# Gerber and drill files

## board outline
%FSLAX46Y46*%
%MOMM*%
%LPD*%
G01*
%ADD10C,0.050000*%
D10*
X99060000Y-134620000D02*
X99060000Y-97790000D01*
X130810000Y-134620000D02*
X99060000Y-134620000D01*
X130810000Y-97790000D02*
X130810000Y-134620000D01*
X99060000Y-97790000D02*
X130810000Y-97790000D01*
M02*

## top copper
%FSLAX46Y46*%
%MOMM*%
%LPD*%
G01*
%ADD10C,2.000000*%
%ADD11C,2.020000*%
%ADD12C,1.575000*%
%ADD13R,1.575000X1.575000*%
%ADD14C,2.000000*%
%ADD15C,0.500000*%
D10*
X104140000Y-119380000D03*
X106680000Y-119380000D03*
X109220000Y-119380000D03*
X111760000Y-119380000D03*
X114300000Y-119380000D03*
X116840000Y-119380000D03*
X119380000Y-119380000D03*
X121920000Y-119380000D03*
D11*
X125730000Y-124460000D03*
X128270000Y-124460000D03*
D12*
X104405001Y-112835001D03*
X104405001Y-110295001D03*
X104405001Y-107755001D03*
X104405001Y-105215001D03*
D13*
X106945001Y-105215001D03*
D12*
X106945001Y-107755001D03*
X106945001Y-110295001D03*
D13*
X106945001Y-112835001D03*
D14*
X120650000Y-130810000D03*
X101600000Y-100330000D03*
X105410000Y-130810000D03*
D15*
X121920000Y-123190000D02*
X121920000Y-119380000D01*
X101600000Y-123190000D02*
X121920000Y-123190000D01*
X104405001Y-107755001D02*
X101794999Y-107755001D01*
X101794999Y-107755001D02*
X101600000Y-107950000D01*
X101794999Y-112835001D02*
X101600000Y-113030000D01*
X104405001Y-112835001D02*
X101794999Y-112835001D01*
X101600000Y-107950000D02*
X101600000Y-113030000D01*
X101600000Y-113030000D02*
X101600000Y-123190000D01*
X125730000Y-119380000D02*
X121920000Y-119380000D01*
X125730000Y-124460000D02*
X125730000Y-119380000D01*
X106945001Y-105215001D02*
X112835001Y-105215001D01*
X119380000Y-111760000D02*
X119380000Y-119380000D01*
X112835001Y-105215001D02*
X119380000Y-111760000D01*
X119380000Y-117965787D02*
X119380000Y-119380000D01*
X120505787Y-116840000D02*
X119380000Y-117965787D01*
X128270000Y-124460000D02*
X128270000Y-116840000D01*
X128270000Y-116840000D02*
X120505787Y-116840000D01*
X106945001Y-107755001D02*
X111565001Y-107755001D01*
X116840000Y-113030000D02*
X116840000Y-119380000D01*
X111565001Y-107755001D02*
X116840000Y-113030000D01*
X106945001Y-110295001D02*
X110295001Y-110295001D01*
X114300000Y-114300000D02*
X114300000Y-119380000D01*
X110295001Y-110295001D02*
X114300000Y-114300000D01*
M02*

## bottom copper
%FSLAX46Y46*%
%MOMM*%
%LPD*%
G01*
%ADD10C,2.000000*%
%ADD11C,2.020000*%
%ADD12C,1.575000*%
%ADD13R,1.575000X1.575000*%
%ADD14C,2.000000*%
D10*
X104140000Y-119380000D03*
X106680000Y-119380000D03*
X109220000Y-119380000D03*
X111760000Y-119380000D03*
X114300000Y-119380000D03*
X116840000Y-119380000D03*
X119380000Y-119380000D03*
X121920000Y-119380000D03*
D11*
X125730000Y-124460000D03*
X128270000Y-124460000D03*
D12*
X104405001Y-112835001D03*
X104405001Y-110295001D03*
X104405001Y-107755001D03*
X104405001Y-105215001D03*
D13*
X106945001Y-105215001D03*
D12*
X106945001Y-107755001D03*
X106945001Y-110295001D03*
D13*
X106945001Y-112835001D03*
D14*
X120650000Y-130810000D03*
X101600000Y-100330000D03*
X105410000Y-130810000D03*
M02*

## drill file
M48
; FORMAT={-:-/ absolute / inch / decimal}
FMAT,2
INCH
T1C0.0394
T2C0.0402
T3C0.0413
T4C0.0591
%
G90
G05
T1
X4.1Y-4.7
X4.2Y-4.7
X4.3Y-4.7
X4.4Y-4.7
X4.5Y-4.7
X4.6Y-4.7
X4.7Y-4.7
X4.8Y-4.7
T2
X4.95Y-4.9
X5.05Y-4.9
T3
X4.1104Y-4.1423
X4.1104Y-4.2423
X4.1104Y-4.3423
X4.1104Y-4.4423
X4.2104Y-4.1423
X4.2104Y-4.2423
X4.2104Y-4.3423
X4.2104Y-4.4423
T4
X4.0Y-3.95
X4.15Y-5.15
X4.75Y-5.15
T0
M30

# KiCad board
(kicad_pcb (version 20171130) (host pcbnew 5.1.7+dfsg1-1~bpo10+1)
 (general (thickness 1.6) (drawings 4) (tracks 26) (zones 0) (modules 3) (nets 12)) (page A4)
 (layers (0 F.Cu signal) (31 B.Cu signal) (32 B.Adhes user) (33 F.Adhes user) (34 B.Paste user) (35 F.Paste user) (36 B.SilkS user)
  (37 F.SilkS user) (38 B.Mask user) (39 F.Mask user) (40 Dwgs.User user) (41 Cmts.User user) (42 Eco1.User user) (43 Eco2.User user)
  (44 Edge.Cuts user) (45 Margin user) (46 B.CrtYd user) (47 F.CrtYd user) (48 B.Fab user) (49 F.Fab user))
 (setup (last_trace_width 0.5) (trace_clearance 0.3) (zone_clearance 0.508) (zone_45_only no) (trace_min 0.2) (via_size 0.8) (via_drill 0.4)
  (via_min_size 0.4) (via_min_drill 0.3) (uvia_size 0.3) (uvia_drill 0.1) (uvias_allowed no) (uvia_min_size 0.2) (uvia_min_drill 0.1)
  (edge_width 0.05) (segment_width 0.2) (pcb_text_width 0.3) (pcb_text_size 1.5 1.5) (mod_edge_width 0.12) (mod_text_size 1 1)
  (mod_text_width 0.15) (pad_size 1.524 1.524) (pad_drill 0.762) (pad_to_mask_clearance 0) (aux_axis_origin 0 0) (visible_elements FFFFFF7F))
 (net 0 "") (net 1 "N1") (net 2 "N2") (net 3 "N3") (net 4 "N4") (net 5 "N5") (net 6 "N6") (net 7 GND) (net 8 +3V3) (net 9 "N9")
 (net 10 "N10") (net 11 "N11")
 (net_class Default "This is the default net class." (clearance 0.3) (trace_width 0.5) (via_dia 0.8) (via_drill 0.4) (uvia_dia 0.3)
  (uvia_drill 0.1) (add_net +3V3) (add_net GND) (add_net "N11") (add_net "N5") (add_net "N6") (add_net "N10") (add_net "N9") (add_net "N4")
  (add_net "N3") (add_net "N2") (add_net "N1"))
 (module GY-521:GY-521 (layer F.Cu) (at 113.03 125.73 180)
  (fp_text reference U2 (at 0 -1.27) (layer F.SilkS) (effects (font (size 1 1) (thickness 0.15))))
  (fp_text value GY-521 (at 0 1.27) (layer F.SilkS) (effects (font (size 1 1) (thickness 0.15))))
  (pad 8 thru_hole circle (at 8.89 6.35 180) (size 2 2) (drill 1) (layers *.Cu *.Mask F.SilkS) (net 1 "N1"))
  (pad 7 thru_hole circle (at 6.35 6.35 180) (size 2 2) (drill 1) (layers *.Cu *.Mask F.SilkS) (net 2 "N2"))
  (pad 6 thru_hole circle (at 3.81 6.35 180) (size 2 2) (drill 1) (layers *.Cu *.Mask F.SilkS) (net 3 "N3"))
  (pad 5 thru_hole circle (at 1.27 6.35 180) (size 2 2) (drill 1) (layers *.Cu *.Mask F.SilkS) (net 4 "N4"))
  (pad 4 thru_hole circle (at -1.27 6.35 180) (size 2 2) (drill 1) (layers *.Cu *.Mask F.SilkS) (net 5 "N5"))
  (pad 3 thru_hole circle (at -3.81 6.35 180) (size 2 2) (drill 1) (layers *.Cu *.Mask F.SilkS) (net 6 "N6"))
  (pad 2 thru_hole circle (at -6.35 6.35 180) (size 2 2) (drill 1) (layers *.Cu *.Mask F.SilkS) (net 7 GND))
  (pad 1 thru_hole circle (at -8.89 6.35 180) (size 2 2) (drill 1) (layers *.Cu *.Mask F.SilkS) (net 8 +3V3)))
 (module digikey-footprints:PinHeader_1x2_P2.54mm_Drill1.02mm (layer F.Cu) (at 128.27 124.46 180)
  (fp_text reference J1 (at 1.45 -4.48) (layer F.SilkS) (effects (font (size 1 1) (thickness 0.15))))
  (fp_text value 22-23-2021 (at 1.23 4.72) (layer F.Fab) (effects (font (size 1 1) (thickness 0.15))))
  (pad 2 thru_hole circle (at 2.54 0 180) (size 2.02 2.02) (drill 1.02) (layers *.Cu *.Mask) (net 8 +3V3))
  (pad 1 thru_hole circle (at 0 0 180) (size 2.02 2.02) (drill 1.02) (layers *.Cu *.Mask) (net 7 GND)))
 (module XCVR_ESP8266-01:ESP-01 (layer F.Cu) (at 106.945001 109.025001)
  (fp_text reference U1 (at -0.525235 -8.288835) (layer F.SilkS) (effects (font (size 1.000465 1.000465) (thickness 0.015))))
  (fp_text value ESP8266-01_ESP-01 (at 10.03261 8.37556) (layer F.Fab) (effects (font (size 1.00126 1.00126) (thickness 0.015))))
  (pad 8 thru_hole circle (at -2.54 3.81) (size 1.575 1.575) (drill 1.05) (layers *.Cu *.Mask) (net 8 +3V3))
  (pad 7 thru_hole circle (at -2.54 1.27) (size 1.575 1.575) (drill 1.05) (layers *.Cu *.Mask) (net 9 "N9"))
  (pad 6 thru_hole circle (at -2.54 -1.27) (size 1.575 1.575) (drill 1.05) (layers *.Cu *.Mask) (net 8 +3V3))
  (pad 5 thru_hole circle (at -2.54 -3.81) (size 1.575 1.575) (drill 1.05) (layers *.Cu *.Mask) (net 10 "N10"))
  (pad 4 thru_hole rect (at 0 -3.81) (size 1.575 1.575) (drill 1.05) (layers *.Cu *.Mask) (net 7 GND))
  (pad 3 thru_hole circle (at 0 -1.27) (size 1.575 1.575) (drill 1.05) (layers *.Cu *.Mask) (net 6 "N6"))
  (pad 2 thru_hole circle (at 0 1.27) (size 1.575 1.575) (drill 1.05) (layers *.Cu *.Mask) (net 5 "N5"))
  (pad 1 thru_hole rect (at 0 3.81) (size 1.575 1.575) (drill 1.05) (layers *.Cu *.Mask) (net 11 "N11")))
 (gr_line (start 99.06 134.62) (end 99.06 97.79) (layer Edge.Cuts) (width 0.05))
 (gr_line (start 130.81 134.62) (end 99.06 134.62) (layer Edge.Cuts) (width 0.05))
 (gr_line (start 130.81 97.79) (end 130.81 134.62) (layer Edge.Cuts) (width 0.05))
 (gr_line (start 99.06 97.79) (end 130.81 97.79) (layer Edge.Cuts) (width 0.05))
 (via (at 120.65 130.81) (size 2) (drill 1.5) (layers F.Cu B.Cu) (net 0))
 (via (at 101.6 100.33) (size 2) (drill 1.5) (layers F.Cu B.Cu) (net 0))
 (via (at 105.41 130.81) (size 2) (drill 1.5) (layers F.Cu B.Cu) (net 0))
 (segment (start 121.92 123.19) (end 121.92 119.38) (width 0.5) (layer F.Cu) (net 8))
 (segment (start 101.6 123.19) (end 121.92 123.19) (width 0.5) (layer F.Cu) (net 8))
 (segment (start 104.405001 107.755001) (end 101.794999 107.755001) (width 0.5) (layer F.Cu) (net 8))
 (segment (start 101.794999 107.755001) (end 101.6 107.95) (width 0.5) (layer F.Cu) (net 8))
 (segment (start 101.794999 112.835001) (end 101.6 113.03) (width 0.5) (layer F.Cu) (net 8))
 (segment (start 104.405001 112.835001) (end 101.794999 112.835001) (width 0.5) (layer F.Cu) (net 8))
 (segment (start 101.6 107.95) (end 101.6 113.03) (width 0.5) (layer F.Cu) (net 8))
 (segment (start 101.6 113.03) (end 101.6 123.19) (width 0.5) (layer F.Cu) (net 8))
 (segment (start 125.73 119.38) (end 121.92 119.38) (width 0.5) (layer F.Cu) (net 8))
 (segment (start 125.73 124.46) (end 125.73 119.38) (width 0.5) (layer F.Cu) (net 8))
 (segment (start 106.945001 105.215001) (end 112.835001 105.215001) (width 0.5) (layer F.Cu) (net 7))
 (segment (start 119.38 111.76) (end 119.38 119.38) (width 0.5) (layer F.Cu) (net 7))
 (segment (start 112.835001 105.215001) (end 119.38 111.76) (width 0.5) (layer F.Cu) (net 7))
 (segment (start 119.38 117.965787) (end 119.38 119.38) (width 0.5) (layer F.Cu) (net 7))
 (segment (start 120.505787 116.84) (end 119.38 117.965787) (width 0.5) (layer F.Cu) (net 7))
 (segment (start 128.27 124.46) (end 128.27 116.84) (width 0.5) (layer F.Cu) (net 7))
 (segment (start 128.27 116.84) (end 120.505787 116.84) (width 0.5) (layer F.Cu) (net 7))
 (segment (start 106.945001 107.755001) (end 111.565001 107.755001) (width 0.5) (layer F.Cu) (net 6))
 (segment (start 116.84 113.03) (end 116.84 119.38) (width 0.5) (layer F.Cu) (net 6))
 (segment (start 111.565001 107.755001) (end 116.84 113.03) (width 0.5) (layer F.Cu) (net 6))
 (segment (start 106.945001 110.295001) (end 110.295001 110.295001) (width 0.5) (layer F.Cu) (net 5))
 (segment (start 114.3 114.3) (end 114.3 119.38) (width 0.5) (layer F.Cu) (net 5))
 (segment (start 110.295001 110.295001) (end 114.3 114.3) (width 0.5) (layer F.Cu) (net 5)))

